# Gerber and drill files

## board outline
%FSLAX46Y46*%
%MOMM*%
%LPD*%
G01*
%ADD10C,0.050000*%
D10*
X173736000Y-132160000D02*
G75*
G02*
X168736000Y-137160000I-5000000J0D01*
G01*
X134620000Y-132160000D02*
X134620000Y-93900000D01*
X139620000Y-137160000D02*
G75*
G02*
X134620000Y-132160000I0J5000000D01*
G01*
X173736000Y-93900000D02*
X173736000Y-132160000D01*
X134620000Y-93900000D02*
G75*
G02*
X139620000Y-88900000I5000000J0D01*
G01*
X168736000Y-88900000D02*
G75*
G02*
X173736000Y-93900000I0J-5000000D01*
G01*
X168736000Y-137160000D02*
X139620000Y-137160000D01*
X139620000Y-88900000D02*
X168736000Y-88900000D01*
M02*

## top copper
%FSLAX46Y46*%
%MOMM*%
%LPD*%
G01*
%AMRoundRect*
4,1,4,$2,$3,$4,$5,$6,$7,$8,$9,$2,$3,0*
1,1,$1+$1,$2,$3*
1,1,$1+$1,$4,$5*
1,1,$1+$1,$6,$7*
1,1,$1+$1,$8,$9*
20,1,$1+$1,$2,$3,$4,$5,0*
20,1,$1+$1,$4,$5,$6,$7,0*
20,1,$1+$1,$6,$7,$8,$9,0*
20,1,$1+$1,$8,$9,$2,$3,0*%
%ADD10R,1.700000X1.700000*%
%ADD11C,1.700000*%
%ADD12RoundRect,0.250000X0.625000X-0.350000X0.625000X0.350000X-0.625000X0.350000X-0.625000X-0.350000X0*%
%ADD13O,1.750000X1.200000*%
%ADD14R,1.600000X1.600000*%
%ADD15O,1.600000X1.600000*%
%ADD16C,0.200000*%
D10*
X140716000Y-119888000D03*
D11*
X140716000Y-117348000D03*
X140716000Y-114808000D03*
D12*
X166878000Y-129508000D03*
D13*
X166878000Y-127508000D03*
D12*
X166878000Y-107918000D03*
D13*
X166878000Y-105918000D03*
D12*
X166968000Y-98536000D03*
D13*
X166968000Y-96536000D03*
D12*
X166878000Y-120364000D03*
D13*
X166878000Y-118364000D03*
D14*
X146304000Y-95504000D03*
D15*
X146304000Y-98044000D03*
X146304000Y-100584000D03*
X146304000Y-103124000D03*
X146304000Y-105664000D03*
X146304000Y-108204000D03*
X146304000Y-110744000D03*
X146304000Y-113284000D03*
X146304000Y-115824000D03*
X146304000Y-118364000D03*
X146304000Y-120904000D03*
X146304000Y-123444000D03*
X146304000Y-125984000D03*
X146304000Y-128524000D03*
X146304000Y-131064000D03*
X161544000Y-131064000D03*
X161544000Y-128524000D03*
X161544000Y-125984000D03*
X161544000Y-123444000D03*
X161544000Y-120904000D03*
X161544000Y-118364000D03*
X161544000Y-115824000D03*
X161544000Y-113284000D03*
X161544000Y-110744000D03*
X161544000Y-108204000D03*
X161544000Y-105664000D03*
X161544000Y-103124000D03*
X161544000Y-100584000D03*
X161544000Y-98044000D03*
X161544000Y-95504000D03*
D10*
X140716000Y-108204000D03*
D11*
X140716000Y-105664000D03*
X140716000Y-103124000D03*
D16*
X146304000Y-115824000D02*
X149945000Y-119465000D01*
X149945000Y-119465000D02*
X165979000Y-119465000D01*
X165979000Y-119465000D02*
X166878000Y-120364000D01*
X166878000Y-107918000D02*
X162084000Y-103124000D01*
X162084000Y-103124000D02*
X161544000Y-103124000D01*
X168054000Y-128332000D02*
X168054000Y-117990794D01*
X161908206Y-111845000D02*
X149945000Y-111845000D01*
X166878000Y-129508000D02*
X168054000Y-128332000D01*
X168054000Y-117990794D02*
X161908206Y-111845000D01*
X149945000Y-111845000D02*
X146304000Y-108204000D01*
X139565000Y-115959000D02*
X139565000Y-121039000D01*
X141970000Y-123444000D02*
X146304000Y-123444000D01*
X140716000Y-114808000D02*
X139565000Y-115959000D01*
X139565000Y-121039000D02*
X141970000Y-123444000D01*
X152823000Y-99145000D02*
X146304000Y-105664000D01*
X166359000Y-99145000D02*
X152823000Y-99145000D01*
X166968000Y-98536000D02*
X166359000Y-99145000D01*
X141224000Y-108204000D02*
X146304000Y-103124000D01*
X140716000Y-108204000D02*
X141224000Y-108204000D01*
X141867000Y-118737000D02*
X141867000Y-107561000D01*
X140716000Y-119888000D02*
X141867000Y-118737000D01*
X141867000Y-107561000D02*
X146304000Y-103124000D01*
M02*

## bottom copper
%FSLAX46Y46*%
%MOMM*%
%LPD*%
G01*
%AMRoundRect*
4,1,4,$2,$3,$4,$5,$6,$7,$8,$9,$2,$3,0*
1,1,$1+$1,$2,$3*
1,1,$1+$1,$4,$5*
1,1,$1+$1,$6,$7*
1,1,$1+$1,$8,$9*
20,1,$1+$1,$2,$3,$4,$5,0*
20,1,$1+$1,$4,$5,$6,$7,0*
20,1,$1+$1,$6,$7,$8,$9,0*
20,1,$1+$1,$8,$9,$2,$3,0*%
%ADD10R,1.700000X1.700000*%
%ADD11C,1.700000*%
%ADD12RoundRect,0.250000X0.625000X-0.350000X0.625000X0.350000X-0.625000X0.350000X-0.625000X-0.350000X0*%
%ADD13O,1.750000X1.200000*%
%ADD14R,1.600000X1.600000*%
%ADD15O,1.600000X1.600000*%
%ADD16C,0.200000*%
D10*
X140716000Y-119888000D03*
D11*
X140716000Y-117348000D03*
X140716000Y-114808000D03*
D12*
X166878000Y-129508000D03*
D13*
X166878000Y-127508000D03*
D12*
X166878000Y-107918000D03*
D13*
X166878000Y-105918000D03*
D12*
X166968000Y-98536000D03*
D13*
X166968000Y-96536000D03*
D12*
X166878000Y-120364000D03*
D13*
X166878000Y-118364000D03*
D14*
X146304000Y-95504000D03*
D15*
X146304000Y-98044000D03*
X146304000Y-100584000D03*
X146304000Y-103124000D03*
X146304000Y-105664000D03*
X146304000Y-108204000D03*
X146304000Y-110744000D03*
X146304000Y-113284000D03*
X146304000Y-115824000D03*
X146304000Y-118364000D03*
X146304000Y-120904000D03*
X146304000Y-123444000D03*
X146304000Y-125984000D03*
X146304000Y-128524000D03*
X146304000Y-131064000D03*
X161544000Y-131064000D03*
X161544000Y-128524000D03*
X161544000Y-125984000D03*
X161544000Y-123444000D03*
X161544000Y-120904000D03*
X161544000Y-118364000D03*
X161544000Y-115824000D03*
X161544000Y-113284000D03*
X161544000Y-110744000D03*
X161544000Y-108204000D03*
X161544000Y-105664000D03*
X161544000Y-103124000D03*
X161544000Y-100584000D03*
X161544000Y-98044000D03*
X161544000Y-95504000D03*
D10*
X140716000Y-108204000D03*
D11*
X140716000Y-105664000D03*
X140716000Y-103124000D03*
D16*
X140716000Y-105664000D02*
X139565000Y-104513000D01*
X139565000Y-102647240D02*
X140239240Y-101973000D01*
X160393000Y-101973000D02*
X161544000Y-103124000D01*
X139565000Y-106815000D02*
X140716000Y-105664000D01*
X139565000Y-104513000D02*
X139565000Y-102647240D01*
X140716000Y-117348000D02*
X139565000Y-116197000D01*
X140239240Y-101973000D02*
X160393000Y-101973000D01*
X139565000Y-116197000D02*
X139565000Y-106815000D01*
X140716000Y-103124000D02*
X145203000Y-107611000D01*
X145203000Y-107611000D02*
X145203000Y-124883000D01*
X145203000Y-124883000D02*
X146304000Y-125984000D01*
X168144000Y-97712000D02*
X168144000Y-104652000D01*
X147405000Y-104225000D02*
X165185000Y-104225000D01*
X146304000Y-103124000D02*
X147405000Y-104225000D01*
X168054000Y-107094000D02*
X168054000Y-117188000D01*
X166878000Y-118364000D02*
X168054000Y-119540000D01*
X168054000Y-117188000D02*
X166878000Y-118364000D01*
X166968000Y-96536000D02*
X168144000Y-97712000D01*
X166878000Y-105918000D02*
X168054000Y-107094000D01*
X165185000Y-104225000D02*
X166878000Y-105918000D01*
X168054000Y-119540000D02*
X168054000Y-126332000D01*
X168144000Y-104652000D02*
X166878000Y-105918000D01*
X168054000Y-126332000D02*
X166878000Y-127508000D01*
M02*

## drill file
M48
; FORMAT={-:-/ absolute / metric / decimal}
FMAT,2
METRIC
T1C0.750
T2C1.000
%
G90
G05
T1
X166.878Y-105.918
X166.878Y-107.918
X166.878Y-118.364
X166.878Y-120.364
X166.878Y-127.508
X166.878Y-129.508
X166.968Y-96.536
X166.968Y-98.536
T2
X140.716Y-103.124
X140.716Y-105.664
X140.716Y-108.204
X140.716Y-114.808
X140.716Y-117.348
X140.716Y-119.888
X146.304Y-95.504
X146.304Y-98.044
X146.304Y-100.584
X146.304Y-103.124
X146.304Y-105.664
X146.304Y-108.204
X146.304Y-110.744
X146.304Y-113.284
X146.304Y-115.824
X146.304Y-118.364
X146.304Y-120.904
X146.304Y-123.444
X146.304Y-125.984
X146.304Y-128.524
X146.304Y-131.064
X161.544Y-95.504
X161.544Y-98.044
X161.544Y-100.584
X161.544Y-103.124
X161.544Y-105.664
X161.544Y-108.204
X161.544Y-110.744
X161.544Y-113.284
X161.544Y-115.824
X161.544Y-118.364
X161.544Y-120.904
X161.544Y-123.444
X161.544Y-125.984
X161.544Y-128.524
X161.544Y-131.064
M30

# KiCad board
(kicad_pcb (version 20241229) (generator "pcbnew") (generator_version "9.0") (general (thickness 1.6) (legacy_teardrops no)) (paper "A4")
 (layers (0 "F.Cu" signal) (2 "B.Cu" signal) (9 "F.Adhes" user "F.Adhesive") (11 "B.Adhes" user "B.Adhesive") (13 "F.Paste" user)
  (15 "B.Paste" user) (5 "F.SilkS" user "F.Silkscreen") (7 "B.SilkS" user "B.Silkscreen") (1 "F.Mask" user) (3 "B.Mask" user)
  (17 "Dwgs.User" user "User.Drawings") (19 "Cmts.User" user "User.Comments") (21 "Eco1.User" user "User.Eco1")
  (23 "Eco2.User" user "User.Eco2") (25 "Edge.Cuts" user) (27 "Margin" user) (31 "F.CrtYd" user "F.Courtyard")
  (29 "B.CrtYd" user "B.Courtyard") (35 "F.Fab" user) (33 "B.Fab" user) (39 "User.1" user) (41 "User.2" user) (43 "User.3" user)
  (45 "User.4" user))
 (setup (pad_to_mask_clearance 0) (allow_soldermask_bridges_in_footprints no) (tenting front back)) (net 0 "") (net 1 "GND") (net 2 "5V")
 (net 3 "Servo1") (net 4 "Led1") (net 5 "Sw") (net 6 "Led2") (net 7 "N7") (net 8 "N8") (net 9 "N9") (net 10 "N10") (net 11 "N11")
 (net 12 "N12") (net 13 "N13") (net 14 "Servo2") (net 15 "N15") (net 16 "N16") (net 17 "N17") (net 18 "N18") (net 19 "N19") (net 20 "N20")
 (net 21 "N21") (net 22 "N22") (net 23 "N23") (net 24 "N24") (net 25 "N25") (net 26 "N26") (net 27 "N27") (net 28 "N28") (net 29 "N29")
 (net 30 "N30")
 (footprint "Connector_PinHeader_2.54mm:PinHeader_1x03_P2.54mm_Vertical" (layer "F.Cu") (at 140.716 119.888 180)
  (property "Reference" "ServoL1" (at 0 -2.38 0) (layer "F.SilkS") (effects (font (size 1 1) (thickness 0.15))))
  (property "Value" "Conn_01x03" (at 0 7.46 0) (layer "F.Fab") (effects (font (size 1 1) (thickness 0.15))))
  (pad "1" thru_hole rect (at 0 0 180) (size 1.7 1.7) (drill 1) (layers "*.Cu" "*.Mask") (remove_unused_layers no) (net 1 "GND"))
  (pad "2" thru_hole circle (at 0 2.54 180) (size 1.7 1.7) (drill 1) (layers "*.Cu" "*.Mask") (remove_unused_layers no) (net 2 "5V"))
  (pad "3" thru_hole circle (at 0 5.08 180) (size 1.7 1.7) (drill 1) (layers "*.Cu" "*.Mask") (remove_unused_layers no) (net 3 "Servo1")))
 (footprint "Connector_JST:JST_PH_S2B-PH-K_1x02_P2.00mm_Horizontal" (layer "F.Cu") (at 166.878 129.508 90)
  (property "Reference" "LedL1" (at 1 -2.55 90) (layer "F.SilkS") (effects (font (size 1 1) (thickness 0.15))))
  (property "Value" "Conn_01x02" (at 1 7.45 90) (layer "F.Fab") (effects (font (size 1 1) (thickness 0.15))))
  (pad "1" thru_hole roundrect (at 0 0 90) (size 1.2 1.75) (drill 0.75) (layers "*.Cu" "*.Mask") (remove_unused_layers no)
   (roundrect_rratio 0.208333) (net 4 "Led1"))
  (pad "2" thru_hole oval (at 2 0 90) (size 1.2 1.75) (drill 0.75) (layers "*.Cu" "*.Mask") (remove_unused_layers no) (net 1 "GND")))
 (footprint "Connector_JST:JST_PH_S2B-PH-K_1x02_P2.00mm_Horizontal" (layer "F.Cu") (at 166.878 107.918 90)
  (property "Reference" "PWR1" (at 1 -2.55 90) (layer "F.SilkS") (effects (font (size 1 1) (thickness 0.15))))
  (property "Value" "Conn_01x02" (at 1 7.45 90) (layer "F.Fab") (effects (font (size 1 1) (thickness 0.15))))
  (pad "1" thru_hole roundrect (at 0 0 90) (size 1.2 1.75) (drill 0.75) (layers "*.Cu" "*.Mask") (remove_unused_layers no)
   (roundrect_rratio 0.208333) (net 2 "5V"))
  (pad "2" thru_hole oval (at 2 0 90) (size 1.2 1.75) (drill 0.75) (layers "*.Cu" "*.Mask") (remove_unused_layers no) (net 1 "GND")))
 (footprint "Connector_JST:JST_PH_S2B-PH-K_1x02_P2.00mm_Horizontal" (layer "F.Cu") (at 166.968 98.536 90)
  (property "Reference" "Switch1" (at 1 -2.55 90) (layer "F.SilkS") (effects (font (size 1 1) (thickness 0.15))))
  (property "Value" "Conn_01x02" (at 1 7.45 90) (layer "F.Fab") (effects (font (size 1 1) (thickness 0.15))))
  (pad "1" thru_hole roundrect (at 0 0 90) (size 1.2 1.75) (drill 0.75) (layers "*.Cu" "*.Mask") (remove_unused_layers no)
   (roundrect_rratio 0.208333) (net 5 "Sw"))
  (pad "2" thru_hole oval (at 2 0 90) (size 1.2 1.75) (drill 0.75) (layers "*.Cu" "*.Mask") (remove_unused_layers no) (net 1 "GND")))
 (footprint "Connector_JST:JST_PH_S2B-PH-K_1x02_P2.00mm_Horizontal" (layer "F.Cu") (at 166.878 120.364 90)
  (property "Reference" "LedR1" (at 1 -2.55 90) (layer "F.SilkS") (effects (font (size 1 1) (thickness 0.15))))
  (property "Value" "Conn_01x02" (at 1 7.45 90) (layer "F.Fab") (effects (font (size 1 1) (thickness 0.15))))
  (pad "1" thru_hole roundrect (at 0 0 90) (size 1.2 1.75) (drill 0.75) (layers "*.Cu" "*.Mask") (remove_unused_layers no)
   (roundrect_rratio 0.208333) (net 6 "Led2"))
  (pad "2" thru_hole oval (at 2 0 90) (size 1.2 1.75) (drill 0.75) (layers "*.Cu" "*.Mask") (remove_unused_layers no) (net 1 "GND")))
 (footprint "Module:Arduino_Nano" (layer "F.Cu") (at 146.304 95.504)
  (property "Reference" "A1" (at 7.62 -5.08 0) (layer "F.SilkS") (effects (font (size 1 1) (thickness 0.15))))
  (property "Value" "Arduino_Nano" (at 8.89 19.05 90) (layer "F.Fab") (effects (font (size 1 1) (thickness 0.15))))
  (pad "1" thru_hole rect (at 0 0) (size 1.6 1.6) (drill 1) (layers "*.Cu" "*.Mask") (remove_unused_layers no) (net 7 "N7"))
  (pad "2" thru_hole oval (at 0 2.54) (size 1.6 1.6) (drill 1) (layers "*.Cu" "*.Mask") (remove_unused_layers no) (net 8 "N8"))
  (pad "3" thru_hole oval (at 0 5.08) (size 1.6 1.6) (drill 1) (layers "*.Cu" "*.Mask") (remove_unused_layers no) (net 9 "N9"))
  (pad "4" thru_hole oval (at 0 7.62) (size 1.6 1.6) (drill 1) (layers "*.Cu" "*.Mask") (remove_unused_layers no) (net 1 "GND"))
  (pad "5" thru_hole oval (at 0 10.16) (size 1.6 1.6) (drill 1) (layers "*.Cu" "*.Mask") (remove_unused_layers no) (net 5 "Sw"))
  (pad "6" thru_hole oval (at 0 12.7) (size 1.6 1.6) (drill 1) (layers "*.Cu" "*.Mask") (remove_unused_layers no) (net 4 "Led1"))
  (pad "7" thru_hole oval (at 0 15.24) (size 1.6 1.6) (drill 1) (layers "*.Cu" "*.Mask") (remove_unused_layers no) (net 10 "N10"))
  (pad "8" thru_hole oval (at 0 17.78) (size 1.6 1.6) (drill 1) (layers "*.Cu" "*.Mask") (remove_unused_layers no) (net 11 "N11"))
  (pad "9" thru_hole oval (at 0 20.32) (size 1.6 1.6) (drill 1) (layers "*.Cu" "*.Mask") (remove_unused_layers no) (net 6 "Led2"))
  (pad "10" thru_hole oval (at 0 22.86) (size 1.6 1.6) (drill 1) (layers "*.Cu" "*.Mask") (remove_unused_layers no) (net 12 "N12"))
  (pad "11" thru_hole oval (at 0 25.4) (size 1.6 1.6) (drill 1) (layers "*.Cu" "*.Mask") (remove_unused_layers no) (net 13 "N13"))
  (pad "12" thru_hole oval (at 0 27.94) (size 1.6 1.6) (drill 1) (layers "*.Cu" "*.Mask") (remove_unused_layers no) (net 3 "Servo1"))
  (pad "13" thru_hole oval (at 0 30.48) (size 1.6 1.6) (drill 1) (layers "*.Cu" "*.Mask") (remove_unused_layers no) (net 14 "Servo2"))
  (pad "14" thru_hole oval (at 0 33.02) (size 1.6 1.6) (drill 1) (layers "*.Cu" "*.Mask") (remove_unused_layers no) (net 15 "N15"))
  (pad "15" thru_hole oval (at 0 35.56) (size 1.6 1.6) (drill 1) (layers "*.Cu" "*.Mask") (remove_unused_layers no) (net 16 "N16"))
  (pad "16" thru_hole oval (at 15.24 35.56) (size 1.6 1.6) (drill 1) (layers "*.Cu" "*.Mask") (remove_unused_layers no) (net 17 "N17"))
  (pad "17" thru_hole oval (at 15.24 33.02) (size 1.6 1.6) (drill 1) (layers "*.Cu" "*.Mask") (remove_unused_layers no) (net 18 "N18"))
  (pad "18" thru_hole oval (at 15.24 30.48) (size 1.6 1.6) (drill 1) (layers "*.Cu" "*.Mask") (remove_unused_layers no) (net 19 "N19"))
  (pad "19" thru_hole oval (at 15.24 27.94) (size 1.6 1.6) (drill 1) (layers "*.Cu" "*.Mask") (remove_unused_layers no) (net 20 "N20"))
  (pad "20" thru_hole oval (at 15.24 25.4) (size 1.6 1.6) (drill 1) (layers "*.Cu" "*.Mask") (remove_unused_layers no) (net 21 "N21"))
  (pad "21" thru_hole oval (at 15.24 22.86) (size 1.6 1.6) (drill 1) (layers "*.Cu" "*.Mask") (remove_unused_layers no) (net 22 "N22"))
  (pad "22" thru_hole oval (at 15.24 20.32) (size 1.6 1.6) (drill 1) (layers "*.Cu" "*.Mask") (remove_unused_layers no) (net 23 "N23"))
  (pad "23" thru_hole oval (at 15.24 17.78) (size 1.6 1.6) (drill 1) (layers "*.Cu" "*.Mask") (remove_unused_layers no) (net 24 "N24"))
  (pad "24" thru_hole oval (at 15.24 15.24) (size 1.6 1.6) (drill 1) (layers "*.Cu" "*.Mask") (remove_unused_layers no) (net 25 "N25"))
  (pad "25" thru_hole oval (at 15.24 12.7) (size 1.6 1.6) (drill 1) (layers "*.Cu" "*.Mask") (remove_unused_layers no) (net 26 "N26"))
  (pad "26" thru_hole oval (at 15.24 10.16) (size 1.6 1.6) (drill 1) (layers "*.Cu" "*.Mask") (remove_unused_layers no) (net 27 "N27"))
  (pad "27" thru_hole oval (at 15.24 7.62) (size 1.6 1.6) (drill 1) (layers "*.Cu" "*.Mask") (remove_unused_layers no) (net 2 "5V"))
  (pad "28" thru_hole oval (at 15.24 5.08) (size 1.6 1.6) (drill 1) (layers "*.Cu" "*.Mask") (remove_unused_layers no) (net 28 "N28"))
  (pad "29" thru_hole oval (at 15.24 2.54) (size 1.6 1.6) (drill 1) (layers "*.Cu" "*.Mask") (remove_unused_layers no) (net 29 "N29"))
  (pad "30" thru_hole oval (at 15.24 0) (size 1.6 1.6) (drill 1) (layers "*.Cu" "*.Mask") (remove_unused_layers no) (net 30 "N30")))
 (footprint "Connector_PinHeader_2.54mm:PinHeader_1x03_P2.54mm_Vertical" (layer "F.Cu") (at 140.716 108.204 180)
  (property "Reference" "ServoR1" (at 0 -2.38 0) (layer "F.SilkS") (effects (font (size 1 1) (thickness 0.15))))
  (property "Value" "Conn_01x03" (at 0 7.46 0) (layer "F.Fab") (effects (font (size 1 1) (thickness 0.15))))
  (pad "1" thru_hole rect (at 0 0 180) (size 1.7 1.7) (drill 1) (layers "*.Cu" "*.Mask") (remove_unused_layers no) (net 1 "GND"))
  (pad "2" thru_hole circle (at 0 2.54 180) (size 1.7 1.7) (drill 1) (layers "*.Cu" "*.Mask") (remove_unused_layers no) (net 2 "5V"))
  (pad "3" thru_hole circle (at 0 5.08 180) (size 1.7 1.7) (drill 1) (layers "*.Cu" "*.Mask") (remove_unused_layers no) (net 14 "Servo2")))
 (gr_arc (start 173.736 132.16) (mid 172.271534 135.695534) (end 168.736 137.16) (stroke (width 0.05) (type default)) (layer "Edge.Cuts"))
 (gr_line (start 134.62 132.16) (end 134.62 93.9) (stroke (width 0.05) (type default)) (layer "Edge.Cuts"))
 (gr_arc (start 139.62 137.16) (mid 136.084466 135.695534) (end 134.62 132.16) (stroke (width 0.05) (type default)) (layer "Edge.Cuts"))
 (gr_line (start 173.736 93.9) (end 173.736 132.16) (stroke (width 0.05) (type default)) (layer "Edge.Cuts"))
 (gr_arc (start 134.62 93.9) (mid 136.084466 90.364466) (end 139.62 88.9) (stroke (width 0.05) (type default)) (layer "Edge.Cuts"))
 (gr_arc (start 168.736 88.9) (mid 172.271534 90.364466) (end 173.736 93.9) (stroke (width 0.05) (type default)) (layer "Edge.Cuts"))
 (gr_line (start 168.736 137.16) (end 139.62 137.16) (stroke (width 0.05) (type default)) (layer "Edge.Cuts"))
 (gr_line (start 139.62 88.9) (end 168.736 88.9) (stroke (width 0.05) (type default)) (layer "Edge.Cuts"))
 (segment (start 146.304 115.824) (end 149.945 119.465) (width 0.2) (layer "F.Cu") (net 6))
 (segment (start 149.945 119.465) (end 165.979 119.465) (width 0.2) (layer "F.Cu") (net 6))
 (segment (start 165.979 119.465) (end 166.878 120.364) (width 0.2) (layer "F.Cu") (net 6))
 (segment (start 166.878 107.918) (end 162.084 103.124) (width 0.2) (layer "F.Cu") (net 2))
 (segment (start 162.084 103.124) (end 161.544 103.124) (width 0.2) (layer "F.Cu") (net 2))
 (segment (start 140.716 105.664) (end 139.565 104.513) (width 0.2) (layer "B.Cu") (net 2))
 (segment (start 139.565 102.64724) (end 140.23924 101.973) (width 0.2) (layer "B.Cu") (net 2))
 (segment (start 160.393 101.973) (end 161.544 103.124) (width 0.2) (layer "B.Cu") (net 2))
 (segment (start 139.565 106.815) (end 140.716 105.664) (width 0.2) (layer "B.Cu") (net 2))
 (segment (start 139.565 104.513) (end 139.565 102.64724) (width 0.2) (layer "B.Cu") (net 2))
 (segment (start 140.716 117.348) (end 139.565 116.197) (width 0.2) (layer "B.Cu") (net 2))
 (segment (start 140.23924 101.973) (end 160.393 101.973) (width 0.2) (layer "B.Cu") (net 2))
 (segment (start 139.565 116.197) (end 139.565 106.815) (width 0.2) (layer "B.Cu") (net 2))
 (segment (start 168.054 128.332) (end 168.054 117.990794) (width 0.2) (layer "F.Cu") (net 4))
 (segment (start 161.908206 111.845) (end 149.945 111.845) (width 0.2) (layer "F.Cu") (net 4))
 (segment (start 166.878 129.508) (end 168.054 128.332) (width 0.2) (layer "F.Cu") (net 4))
 (segment (start 168.054 117.990794) (end 161.908206 111.845) (width 0.2) (layer "F.Cu") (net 4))
 (segment (start 149.945 111.845) (end 146.304 108.204) (width 0.2) (layer "F.Cu") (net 4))
 (segment (start 140.716 103.124) (end 145.203 107.611) (width 0.2) (layer "B.Cu") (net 14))
 (segment (start 145.203 107.611) (end 145.203 124.883) (width 0.2) (layer "B.Cu") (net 14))
 (segment (start 145.203 124.883) (end 146.304 125.984) (width 0.2) (layer "B.Cu") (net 14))
 (segment (start 139.565 115.959) (end 139.565 121.039) (width 0.2) (layer "F.Cu") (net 3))
 (segment (start 141.97 123.444) (end 146.304 123.444) (width 0.2) (layer "F.Cu") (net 3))
 (segment (start 140.716 114.808) (end 139.565 115.959) (width 0.2) (layer "F.Cu") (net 3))
 (segment (start 139.565 121.039) (end 141.97 123.444) (width 0.2) (layer "F.Cu") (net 3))
 (segment (start 152.823 99.145) (end 146.304 105.664) (width 0.2) (layer "F.Cu") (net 5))
 (segment (start 166.359 99.145) (end 152.823 99.145) (width 0.2) (layer "F.Cu") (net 5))
 (segment (start 166.968 98.536) (end 166.359 99.145) (width 0.2) (layer "F.Cu") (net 5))
 (segment (start 141.224 108.204) (end 146.304 103.124) (width 0.2) (layer "F.Cu") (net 1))
 (segment (start 140.716 108.204) (end 141.224 108.204) (width 0.2) (layer "F.Cu") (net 1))
 (segment (start 141.867 118.737) (end 141.867 107.561) (width 0.2) (layer "F.Cu") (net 1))
 (segment (start 140.716 119.888) (end 141.867 118.737) (width 0.2) (layer "F.Cu") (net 1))
 (segment (start 141.867 107.561) (end 146.304 103.124) (width 0.2) (layer "F.Cu") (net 1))
 (segment (start 168.144 97.712) (end 168.144 104.652) (width 0.2) (layer "B.Cu") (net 1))
 (segment (start 147.405 104.225) (end 165.185 104.225) (width 0.2) (layer "B.Cu") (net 1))
 (segment (start 146.304 103.124) (end 147.405 104.225) (width 0.2) (layer "B.Cu") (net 1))
 (segment (start 168.054 107.094) (end 168.054 117.188) (width 0.2) (layer "B.Cu") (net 1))
 (segment (start 166.878 118.364) (end 168.054 119.54) (width 0.2) (layer "B.Cu") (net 1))
 (segment (start 168.054 117.188) (end 166.878 118.364) (width 0.2) (layer "B.Cu") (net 1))
 (segment (start 166.968 96.536) (end 168.144 97.712) (width 0.2) (layer "B.Cu") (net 1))
 (segment (start 166.878 105.918) (end 168.054 107.094) (width 0.2) (layer "B.Cu") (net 1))
 (segment (start 165.185 104.225) (end 166.878 105.918) (width 0.2) (layer "B.Cu") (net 1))
 (segment (start 168.054 119.54) (end 168.054 126.332) (width 0.2) (layer "B.Cu") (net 1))
 (segment (start 168.144 104.652) (end 166.878 105.918) (width 0.2) (layer "B.Cu") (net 1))
 (segment (start 168.054 126.332) (end 166.878 127.508) (width 0.2) (layer "B.Cu") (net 1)))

